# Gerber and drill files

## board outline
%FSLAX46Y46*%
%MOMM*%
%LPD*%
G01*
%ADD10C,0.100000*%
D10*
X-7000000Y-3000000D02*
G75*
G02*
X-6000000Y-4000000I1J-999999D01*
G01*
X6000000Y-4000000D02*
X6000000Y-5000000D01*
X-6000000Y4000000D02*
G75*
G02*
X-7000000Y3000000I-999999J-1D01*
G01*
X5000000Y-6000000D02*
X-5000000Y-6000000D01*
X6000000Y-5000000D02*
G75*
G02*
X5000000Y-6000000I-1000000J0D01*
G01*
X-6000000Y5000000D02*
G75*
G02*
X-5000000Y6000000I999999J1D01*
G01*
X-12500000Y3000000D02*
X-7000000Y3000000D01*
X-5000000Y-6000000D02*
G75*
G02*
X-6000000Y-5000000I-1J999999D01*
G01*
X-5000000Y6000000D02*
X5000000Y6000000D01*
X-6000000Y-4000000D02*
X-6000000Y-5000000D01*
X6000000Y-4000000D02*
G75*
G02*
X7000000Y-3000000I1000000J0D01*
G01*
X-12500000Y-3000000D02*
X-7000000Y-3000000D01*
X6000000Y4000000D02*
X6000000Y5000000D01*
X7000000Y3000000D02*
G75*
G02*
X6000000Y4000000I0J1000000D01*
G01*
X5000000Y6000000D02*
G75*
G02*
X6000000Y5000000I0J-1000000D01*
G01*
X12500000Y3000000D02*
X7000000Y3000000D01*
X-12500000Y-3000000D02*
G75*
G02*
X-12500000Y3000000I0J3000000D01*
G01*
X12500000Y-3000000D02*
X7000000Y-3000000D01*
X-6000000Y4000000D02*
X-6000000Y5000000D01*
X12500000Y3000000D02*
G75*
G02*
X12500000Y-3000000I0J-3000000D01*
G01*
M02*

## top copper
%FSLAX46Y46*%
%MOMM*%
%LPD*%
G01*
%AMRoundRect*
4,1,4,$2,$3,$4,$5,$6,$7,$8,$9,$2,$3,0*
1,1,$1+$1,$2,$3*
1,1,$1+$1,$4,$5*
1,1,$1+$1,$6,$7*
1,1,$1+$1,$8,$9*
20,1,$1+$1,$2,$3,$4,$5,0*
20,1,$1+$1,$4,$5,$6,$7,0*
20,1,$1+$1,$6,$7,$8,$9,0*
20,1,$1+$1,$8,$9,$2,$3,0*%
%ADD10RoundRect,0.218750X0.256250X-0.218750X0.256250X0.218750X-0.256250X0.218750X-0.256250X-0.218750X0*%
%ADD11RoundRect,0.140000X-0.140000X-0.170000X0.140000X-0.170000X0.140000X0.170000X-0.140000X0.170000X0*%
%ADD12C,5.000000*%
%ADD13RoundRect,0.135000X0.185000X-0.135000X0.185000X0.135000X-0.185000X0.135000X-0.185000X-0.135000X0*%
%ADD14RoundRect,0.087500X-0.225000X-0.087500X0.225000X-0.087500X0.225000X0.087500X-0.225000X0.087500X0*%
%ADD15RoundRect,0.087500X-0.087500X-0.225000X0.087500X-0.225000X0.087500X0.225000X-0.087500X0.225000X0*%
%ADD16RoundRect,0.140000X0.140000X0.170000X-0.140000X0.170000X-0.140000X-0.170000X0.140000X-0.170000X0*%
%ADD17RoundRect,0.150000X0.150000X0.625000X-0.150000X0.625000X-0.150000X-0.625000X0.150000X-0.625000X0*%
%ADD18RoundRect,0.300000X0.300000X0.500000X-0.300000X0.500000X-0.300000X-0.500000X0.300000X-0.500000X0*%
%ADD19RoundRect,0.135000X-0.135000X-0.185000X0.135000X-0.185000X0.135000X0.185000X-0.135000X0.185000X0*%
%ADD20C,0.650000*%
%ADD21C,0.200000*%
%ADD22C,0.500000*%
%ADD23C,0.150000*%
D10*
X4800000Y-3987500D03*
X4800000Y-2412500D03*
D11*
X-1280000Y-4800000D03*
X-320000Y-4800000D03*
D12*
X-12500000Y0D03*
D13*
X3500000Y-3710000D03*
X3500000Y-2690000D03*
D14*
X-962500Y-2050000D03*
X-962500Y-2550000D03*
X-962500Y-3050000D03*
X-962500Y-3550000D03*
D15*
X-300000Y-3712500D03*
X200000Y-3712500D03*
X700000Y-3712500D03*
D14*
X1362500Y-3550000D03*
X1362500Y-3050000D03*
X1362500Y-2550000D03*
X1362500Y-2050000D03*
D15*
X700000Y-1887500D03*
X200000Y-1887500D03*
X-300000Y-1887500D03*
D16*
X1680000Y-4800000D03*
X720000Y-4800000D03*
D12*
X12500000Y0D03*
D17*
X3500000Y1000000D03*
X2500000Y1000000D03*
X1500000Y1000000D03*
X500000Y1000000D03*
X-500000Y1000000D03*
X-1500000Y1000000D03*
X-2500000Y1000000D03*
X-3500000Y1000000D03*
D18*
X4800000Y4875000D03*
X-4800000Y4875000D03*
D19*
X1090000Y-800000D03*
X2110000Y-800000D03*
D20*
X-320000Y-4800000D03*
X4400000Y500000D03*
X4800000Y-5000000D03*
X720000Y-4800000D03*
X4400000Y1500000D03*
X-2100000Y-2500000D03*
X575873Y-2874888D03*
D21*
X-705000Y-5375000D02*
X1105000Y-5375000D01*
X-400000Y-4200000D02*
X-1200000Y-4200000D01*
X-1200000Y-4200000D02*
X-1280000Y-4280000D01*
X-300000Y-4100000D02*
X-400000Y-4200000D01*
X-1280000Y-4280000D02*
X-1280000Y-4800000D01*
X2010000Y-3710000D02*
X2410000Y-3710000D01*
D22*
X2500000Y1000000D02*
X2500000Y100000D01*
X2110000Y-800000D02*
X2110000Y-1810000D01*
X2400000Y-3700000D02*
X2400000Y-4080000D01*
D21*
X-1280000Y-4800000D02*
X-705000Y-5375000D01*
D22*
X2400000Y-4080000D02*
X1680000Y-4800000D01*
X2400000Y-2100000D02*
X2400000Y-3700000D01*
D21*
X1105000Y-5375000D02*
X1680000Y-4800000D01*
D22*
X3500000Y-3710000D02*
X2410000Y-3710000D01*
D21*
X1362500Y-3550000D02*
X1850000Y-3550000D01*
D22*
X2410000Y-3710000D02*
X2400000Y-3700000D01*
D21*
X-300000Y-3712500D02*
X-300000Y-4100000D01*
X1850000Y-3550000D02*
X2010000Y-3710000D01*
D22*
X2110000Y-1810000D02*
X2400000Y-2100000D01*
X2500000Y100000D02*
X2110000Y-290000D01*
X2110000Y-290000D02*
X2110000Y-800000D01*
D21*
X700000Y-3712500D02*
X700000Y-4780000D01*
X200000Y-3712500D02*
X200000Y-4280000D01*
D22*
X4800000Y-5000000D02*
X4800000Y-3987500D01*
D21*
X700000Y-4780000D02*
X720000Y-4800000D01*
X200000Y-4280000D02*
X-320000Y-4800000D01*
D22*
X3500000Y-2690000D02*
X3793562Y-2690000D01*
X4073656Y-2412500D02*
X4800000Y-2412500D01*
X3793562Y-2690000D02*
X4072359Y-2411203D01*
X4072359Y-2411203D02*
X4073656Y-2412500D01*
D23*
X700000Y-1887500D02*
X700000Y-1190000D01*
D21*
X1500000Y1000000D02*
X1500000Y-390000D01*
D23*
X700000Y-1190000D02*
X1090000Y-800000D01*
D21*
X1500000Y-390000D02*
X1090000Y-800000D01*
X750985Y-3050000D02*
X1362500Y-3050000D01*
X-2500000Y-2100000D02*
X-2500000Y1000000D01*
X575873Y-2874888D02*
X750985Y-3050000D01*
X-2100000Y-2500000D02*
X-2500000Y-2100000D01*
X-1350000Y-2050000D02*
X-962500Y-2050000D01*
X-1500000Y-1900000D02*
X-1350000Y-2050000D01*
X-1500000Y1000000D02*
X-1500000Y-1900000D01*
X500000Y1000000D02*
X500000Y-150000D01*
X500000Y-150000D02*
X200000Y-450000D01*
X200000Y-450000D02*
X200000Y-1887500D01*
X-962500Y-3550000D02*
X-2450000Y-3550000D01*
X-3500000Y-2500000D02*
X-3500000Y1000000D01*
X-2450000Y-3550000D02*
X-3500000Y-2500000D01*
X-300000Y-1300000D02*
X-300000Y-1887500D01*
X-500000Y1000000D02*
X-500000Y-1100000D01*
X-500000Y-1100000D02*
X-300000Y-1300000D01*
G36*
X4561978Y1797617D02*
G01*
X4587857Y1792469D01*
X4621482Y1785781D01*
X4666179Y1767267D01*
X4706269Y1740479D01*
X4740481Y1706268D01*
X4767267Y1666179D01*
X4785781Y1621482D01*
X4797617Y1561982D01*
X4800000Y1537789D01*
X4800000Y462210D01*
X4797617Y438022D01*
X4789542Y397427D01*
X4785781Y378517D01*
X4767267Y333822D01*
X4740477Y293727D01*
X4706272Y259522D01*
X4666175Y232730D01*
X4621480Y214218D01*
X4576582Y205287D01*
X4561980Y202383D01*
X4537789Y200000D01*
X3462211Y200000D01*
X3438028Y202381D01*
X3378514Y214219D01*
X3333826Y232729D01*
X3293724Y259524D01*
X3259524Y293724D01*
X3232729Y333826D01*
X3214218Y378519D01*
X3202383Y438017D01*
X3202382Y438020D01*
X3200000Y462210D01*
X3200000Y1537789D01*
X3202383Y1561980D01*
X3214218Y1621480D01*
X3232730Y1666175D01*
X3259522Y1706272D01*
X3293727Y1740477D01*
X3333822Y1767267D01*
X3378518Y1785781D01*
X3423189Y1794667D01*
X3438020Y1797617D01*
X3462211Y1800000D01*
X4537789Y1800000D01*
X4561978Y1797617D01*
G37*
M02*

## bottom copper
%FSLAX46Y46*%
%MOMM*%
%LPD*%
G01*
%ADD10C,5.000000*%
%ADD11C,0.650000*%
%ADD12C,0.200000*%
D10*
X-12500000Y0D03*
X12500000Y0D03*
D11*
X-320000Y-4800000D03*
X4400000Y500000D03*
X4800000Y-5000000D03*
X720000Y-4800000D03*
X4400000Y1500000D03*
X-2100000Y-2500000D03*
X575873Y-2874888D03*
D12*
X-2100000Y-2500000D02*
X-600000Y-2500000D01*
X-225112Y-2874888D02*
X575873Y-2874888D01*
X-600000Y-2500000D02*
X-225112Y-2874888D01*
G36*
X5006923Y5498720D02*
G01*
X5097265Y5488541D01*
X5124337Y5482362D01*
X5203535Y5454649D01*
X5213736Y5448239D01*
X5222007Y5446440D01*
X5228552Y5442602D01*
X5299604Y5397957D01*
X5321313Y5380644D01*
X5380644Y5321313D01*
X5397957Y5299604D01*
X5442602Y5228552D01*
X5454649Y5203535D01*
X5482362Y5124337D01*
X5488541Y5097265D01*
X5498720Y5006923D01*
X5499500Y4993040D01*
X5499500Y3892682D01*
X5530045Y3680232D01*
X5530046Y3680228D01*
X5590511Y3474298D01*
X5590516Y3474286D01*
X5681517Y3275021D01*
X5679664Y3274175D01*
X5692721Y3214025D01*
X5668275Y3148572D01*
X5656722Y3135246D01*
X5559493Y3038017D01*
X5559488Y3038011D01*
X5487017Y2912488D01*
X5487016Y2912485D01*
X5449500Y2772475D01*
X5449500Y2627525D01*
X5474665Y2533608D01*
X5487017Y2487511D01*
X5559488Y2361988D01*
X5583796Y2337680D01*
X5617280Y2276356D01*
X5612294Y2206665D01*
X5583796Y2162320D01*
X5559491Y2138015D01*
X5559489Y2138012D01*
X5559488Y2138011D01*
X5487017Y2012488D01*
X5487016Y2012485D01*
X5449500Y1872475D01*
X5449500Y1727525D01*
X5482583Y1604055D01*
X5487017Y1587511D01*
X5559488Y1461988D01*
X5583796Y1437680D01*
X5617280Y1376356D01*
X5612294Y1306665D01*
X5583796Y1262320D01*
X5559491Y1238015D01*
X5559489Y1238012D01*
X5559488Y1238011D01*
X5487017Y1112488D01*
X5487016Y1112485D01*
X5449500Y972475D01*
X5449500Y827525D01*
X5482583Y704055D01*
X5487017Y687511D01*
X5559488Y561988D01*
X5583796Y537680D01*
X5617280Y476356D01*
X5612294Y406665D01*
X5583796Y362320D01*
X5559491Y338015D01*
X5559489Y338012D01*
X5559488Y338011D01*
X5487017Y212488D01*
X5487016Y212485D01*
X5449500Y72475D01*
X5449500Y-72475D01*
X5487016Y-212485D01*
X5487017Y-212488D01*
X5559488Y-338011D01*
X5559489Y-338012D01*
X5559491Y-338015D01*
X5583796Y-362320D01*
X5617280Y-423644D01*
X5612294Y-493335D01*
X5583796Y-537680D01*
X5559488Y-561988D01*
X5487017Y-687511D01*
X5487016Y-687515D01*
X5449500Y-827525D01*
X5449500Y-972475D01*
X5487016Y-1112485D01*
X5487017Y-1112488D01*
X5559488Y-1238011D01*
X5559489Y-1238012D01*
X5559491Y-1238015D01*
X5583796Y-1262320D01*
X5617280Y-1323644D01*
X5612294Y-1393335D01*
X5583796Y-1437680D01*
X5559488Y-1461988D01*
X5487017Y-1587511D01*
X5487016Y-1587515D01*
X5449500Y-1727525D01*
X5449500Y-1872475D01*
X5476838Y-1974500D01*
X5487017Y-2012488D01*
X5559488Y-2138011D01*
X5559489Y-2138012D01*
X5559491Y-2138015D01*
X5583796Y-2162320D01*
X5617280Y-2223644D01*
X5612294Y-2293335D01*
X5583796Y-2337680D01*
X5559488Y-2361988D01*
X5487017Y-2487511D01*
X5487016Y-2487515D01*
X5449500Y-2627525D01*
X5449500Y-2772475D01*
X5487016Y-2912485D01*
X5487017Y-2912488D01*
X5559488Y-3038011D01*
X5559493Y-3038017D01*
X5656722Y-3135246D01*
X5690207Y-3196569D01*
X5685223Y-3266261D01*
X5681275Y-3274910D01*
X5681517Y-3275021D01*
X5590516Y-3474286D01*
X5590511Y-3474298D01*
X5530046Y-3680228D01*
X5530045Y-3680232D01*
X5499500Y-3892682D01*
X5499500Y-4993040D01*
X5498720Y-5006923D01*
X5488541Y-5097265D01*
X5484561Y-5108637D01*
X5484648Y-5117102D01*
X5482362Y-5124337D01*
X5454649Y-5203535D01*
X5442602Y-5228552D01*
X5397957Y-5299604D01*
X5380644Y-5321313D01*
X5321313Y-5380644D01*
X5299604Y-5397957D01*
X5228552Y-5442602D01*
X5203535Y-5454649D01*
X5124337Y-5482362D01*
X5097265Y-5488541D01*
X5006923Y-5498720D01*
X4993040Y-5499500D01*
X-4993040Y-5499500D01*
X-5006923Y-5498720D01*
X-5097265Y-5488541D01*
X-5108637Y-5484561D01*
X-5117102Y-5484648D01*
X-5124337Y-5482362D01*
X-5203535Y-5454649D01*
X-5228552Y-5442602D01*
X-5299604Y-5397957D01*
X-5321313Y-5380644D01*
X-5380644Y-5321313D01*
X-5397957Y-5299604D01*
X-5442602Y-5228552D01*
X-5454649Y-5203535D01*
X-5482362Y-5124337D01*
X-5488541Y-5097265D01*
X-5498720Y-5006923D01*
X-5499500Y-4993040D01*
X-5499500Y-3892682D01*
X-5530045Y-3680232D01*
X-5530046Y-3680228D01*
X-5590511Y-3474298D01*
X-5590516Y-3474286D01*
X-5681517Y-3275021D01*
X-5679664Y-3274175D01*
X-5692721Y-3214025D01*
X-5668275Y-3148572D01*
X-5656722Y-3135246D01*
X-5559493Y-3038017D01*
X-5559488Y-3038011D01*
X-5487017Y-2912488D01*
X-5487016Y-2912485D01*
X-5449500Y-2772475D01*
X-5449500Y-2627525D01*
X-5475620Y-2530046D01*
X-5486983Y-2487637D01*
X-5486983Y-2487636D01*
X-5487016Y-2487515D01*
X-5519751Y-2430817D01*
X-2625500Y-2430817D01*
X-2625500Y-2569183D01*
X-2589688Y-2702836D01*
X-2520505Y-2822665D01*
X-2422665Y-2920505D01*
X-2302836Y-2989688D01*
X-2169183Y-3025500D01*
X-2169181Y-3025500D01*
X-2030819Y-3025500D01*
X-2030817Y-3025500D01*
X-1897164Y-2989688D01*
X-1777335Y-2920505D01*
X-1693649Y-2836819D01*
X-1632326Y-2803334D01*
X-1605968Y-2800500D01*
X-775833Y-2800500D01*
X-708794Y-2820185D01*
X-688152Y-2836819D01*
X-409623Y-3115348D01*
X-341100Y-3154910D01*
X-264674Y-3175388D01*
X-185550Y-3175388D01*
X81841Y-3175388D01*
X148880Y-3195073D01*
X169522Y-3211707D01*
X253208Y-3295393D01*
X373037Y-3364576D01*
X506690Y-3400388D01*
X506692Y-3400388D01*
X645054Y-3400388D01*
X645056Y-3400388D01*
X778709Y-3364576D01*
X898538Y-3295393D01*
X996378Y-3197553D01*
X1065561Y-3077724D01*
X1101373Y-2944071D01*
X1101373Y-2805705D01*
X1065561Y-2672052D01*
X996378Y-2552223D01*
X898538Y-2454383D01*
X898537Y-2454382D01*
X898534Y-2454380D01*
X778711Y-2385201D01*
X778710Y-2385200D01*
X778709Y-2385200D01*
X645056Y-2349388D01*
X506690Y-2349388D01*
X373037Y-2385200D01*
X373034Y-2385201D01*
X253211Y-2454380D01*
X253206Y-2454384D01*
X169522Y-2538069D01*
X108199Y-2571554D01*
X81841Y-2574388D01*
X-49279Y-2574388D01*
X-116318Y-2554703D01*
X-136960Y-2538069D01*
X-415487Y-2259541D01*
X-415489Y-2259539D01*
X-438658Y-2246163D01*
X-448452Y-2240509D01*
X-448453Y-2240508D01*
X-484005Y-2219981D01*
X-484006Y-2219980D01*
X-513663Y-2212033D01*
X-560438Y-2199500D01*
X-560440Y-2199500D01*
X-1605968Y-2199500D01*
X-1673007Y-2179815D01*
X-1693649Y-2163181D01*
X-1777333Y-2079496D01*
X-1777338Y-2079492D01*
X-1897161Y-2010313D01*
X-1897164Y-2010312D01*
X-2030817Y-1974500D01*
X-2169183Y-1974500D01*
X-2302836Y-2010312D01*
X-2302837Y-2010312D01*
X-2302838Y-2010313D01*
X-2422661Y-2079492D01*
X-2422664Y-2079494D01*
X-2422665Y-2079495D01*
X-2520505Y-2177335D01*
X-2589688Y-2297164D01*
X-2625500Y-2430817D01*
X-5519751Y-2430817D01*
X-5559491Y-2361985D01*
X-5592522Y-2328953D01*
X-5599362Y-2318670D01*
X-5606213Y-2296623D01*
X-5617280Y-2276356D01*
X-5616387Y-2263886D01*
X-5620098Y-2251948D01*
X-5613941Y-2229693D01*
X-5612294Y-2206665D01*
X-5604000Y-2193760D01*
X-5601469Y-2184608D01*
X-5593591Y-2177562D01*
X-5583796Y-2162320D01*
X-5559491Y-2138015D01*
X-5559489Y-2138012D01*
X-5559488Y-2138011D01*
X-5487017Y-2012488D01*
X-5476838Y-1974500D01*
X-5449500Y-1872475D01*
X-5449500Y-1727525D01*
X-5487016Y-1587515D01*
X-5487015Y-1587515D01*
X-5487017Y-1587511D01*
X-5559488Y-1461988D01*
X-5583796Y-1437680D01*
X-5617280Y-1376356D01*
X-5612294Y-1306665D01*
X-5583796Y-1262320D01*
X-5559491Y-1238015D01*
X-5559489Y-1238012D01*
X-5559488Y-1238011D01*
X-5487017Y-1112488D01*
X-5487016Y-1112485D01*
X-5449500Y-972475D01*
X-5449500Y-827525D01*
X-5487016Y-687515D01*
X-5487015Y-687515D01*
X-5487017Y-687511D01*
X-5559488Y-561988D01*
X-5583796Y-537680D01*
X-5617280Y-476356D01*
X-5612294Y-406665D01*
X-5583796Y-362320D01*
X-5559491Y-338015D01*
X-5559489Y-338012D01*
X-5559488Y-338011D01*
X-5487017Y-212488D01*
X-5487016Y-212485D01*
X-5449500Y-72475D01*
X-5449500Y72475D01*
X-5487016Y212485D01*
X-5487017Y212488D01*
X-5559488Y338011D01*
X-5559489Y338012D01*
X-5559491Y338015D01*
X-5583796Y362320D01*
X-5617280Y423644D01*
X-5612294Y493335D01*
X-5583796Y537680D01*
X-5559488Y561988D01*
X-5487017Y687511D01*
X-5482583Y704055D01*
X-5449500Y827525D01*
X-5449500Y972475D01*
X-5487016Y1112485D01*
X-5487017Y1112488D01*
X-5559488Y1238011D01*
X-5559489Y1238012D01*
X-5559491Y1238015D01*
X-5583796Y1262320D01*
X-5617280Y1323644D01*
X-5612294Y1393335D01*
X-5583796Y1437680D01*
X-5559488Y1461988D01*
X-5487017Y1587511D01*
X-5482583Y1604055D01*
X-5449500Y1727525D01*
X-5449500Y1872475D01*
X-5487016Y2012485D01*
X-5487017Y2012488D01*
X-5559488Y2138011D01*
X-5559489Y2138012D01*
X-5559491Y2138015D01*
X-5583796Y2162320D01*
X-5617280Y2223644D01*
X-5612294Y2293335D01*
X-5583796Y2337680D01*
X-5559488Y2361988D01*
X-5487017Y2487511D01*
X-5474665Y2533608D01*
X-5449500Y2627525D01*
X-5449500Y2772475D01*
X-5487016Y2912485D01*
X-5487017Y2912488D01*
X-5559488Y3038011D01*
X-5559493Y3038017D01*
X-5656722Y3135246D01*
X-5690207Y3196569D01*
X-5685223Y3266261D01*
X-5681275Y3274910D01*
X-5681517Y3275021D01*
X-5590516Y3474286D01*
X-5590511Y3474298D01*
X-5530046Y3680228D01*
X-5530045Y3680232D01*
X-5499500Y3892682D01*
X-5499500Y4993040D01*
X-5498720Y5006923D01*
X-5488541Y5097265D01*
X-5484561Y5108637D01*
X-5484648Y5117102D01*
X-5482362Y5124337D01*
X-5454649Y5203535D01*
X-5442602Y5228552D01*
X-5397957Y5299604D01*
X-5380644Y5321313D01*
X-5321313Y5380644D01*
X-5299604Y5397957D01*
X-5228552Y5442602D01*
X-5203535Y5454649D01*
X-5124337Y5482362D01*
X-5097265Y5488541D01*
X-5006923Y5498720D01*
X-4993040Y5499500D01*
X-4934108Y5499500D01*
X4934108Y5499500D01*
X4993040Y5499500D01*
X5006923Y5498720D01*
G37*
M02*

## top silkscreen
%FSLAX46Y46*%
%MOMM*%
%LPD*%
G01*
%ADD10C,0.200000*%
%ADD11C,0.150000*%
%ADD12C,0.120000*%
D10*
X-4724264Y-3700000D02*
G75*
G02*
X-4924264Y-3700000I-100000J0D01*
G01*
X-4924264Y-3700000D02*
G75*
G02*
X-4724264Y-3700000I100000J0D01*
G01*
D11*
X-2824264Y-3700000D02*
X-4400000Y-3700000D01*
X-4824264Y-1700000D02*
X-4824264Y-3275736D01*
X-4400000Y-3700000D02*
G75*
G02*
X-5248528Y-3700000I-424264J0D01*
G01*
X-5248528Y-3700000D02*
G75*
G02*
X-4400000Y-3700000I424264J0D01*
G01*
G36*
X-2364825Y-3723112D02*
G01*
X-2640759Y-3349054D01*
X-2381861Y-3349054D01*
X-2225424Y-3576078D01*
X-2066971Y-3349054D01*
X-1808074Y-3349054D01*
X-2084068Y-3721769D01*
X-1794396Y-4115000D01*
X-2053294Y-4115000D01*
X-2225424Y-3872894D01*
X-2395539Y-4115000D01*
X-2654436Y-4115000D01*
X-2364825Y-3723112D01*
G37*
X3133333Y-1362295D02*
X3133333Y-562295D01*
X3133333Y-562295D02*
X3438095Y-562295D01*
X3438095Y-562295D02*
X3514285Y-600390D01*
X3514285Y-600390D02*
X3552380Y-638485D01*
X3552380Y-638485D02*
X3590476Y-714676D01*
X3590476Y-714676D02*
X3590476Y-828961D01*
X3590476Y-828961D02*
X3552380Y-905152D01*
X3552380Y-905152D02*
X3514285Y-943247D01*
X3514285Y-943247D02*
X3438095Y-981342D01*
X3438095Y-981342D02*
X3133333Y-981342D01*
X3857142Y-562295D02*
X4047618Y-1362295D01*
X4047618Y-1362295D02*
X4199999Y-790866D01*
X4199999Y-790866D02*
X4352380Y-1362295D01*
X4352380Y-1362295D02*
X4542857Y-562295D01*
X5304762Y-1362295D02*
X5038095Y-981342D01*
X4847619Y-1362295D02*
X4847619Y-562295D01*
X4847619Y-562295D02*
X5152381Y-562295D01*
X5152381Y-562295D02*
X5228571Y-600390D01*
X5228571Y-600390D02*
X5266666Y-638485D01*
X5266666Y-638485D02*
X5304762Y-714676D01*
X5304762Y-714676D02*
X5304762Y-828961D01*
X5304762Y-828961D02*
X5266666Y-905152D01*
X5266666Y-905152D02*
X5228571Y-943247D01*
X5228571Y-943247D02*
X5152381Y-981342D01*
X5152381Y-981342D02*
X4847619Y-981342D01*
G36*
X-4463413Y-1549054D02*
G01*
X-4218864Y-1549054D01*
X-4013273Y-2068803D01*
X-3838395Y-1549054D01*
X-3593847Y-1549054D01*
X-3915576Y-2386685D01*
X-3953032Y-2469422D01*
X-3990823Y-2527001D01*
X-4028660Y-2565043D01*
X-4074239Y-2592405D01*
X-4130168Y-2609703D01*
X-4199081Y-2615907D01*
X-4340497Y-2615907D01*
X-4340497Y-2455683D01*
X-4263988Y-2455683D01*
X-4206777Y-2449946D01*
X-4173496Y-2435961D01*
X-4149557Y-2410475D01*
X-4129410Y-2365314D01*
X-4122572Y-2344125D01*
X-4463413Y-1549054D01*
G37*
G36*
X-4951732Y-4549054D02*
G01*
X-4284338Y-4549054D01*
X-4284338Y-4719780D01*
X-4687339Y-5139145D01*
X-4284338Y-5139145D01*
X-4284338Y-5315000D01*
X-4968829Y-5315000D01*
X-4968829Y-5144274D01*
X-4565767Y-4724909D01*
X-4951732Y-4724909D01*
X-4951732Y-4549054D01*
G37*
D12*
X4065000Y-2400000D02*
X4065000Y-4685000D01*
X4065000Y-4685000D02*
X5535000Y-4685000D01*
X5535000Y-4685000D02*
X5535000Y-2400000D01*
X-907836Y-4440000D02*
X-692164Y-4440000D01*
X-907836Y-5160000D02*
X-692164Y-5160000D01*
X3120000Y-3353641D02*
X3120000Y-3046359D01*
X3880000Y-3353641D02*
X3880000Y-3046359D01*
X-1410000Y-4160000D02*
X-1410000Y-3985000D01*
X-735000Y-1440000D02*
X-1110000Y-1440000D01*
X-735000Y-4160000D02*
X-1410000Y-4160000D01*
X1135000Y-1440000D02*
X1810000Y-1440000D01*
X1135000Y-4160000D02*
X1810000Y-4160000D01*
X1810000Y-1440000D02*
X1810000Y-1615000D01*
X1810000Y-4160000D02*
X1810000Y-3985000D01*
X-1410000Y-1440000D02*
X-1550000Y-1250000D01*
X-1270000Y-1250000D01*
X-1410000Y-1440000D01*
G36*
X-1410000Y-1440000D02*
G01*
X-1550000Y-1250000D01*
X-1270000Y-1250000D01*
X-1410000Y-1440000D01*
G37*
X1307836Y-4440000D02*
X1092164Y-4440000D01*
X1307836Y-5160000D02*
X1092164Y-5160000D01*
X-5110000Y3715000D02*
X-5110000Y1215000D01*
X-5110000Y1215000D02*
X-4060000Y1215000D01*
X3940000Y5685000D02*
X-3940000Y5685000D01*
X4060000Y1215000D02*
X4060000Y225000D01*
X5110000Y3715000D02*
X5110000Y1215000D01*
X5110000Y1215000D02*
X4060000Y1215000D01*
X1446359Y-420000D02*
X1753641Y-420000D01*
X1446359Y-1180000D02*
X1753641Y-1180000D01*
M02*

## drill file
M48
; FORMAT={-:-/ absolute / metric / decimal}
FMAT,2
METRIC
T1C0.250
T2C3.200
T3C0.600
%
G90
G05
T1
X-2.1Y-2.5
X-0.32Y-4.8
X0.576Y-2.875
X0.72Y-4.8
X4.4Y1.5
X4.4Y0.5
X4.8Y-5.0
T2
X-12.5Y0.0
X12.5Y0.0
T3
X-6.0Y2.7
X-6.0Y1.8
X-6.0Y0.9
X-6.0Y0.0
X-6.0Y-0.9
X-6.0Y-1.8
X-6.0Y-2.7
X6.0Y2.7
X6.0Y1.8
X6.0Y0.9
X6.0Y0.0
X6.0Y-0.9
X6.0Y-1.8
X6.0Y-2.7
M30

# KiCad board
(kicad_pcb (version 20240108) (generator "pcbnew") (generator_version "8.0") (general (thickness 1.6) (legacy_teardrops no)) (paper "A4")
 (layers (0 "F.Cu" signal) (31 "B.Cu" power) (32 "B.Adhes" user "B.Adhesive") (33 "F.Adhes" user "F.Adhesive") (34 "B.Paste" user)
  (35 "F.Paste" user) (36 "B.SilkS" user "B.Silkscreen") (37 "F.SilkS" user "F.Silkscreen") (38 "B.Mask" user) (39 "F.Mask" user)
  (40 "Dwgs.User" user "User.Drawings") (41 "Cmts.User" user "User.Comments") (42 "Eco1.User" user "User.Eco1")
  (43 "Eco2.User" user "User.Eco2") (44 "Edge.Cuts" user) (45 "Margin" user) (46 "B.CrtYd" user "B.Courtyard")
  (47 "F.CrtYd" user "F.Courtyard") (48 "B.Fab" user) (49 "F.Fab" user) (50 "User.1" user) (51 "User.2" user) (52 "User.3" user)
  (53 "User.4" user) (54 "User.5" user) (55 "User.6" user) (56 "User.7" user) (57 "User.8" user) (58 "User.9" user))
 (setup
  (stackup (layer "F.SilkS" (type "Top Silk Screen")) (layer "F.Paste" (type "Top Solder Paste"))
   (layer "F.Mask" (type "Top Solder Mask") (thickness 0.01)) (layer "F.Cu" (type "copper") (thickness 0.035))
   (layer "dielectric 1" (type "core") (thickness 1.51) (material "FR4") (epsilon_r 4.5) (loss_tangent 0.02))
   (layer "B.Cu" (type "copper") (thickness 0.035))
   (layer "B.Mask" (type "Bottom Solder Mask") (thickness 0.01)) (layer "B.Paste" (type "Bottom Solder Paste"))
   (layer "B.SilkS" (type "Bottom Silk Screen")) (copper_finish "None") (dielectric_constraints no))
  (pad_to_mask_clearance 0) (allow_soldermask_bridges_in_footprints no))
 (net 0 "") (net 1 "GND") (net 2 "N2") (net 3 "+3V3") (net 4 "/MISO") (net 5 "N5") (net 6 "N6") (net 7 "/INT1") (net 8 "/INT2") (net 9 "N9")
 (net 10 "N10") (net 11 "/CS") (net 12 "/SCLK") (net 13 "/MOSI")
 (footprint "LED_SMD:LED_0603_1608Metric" (layer "F.Cu") (at 4.8 3.2 90)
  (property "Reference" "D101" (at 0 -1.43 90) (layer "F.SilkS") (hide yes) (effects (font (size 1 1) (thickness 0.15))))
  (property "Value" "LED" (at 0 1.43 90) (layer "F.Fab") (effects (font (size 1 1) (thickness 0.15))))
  (fp_line (start 0.8 -0.735) (end -1.485 -0.735) (stroke (width 0.12) (type solid)) (layer "F.SilkS"))
  (fp_line (start -1.485 -0.735) (end -1.485 0.735) (stroke (width 0.12) (type solid)) (layer "F.SilkS"))
  (fp_line (start -1.485 0.735) (end 0.8 0.735) (stroke (width 0.12) (type solid)) (layer "F.SilkS"))
  (pad "1" smd roundrect (at -0.7875 0 90) (size 0.875 0.95) (layers "F.Cu" "F.Paste" "F.Mask") (roundrect_rratio 0.25) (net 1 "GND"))
  (pad "2" smd roundrect (at 0.7875 0 90) (size 0.875 0.95) (layers "F.Cu" "F.Paste" "F.Mask") (roundrect_rratio 0.25) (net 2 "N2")))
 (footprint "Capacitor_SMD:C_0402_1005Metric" (layer "F.Cu") (at -0.8 4.8)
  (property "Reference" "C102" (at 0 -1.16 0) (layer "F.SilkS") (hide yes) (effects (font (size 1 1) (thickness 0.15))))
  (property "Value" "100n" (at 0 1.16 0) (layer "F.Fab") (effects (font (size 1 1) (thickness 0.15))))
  (fp_line (start -0.107836 -0.36) (end 0.107836 -0.36) (stroke (width 0.12) (type solid)) (layer "F.SilkS"))
  (fp_line (start -0.107836 0.36) (end 0.107836 0.36) (stroke (width 0.12) (type solid)) (layer "F.SilkS"))
  (pad "1" smd roundrect (at -0.48 0) (size 0.56 0.62) (layers "F.Cu" "F.Paste" "F.Mask") (roundrect_rratio 0.25) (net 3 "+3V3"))
  (pad "2" smd roundrect (at 0.48 0) (size 0.56 0.62) (layers "F.Cu" "F.Paste" "F.Mask") (roundrect_rratio 0.25) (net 1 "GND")))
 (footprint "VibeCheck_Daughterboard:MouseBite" (layer "F.Cu") (at -6 0 180)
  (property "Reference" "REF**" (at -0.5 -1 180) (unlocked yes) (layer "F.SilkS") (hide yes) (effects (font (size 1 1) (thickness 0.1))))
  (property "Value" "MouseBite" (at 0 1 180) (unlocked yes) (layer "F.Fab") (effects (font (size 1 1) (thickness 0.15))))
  (pad "" np_thru_hole circle (at 0 -2.7 180) (size 0.6 0.6) (drill 0.6) (layers "F&B.Cu"))
  (pad "" np_thru_hole circle (at 0 -1.8 180) (size 0.6 0.6) (drill 0.6) (layers "F&B.Cu"))
  (pad "" np_thru_hole circle (at 0 -0.9 180) (size 0.6 0.6) (drill 0.6) (layers "F&B.Cu"))
  (pad "" np_thru_hole circle (at 0 0 180) (size 0.6 0.6) (drill 0.6) (layers "F&B.Cu"))
  (pad "" np_thru_hole circle (at 0 0.9 180) (size 0.6 0.6) (drill 0.6) (layers "F&B.Cu"))
  (pad "" np_thru_hole circle (at 0 1.8 180) (size 0.6 0.6) (drill 0.6) (layers "F&B.Cu"))
  (pad "" np_thru_hole circle (at 0 2.7 180) (size 0.6 0.6) (drill 0.6) (layers "F&B.Cu")))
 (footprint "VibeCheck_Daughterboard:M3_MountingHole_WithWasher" (layer "F.Cu") (at -12.5 0)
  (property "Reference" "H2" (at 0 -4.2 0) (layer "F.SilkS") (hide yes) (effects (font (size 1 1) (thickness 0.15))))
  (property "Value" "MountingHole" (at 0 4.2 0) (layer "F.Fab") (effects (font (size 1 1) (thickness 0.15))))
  (pad "1" thru_hole circle (at 0 0) (size 5 5) (drill 3.2) (layers "*.Cu" "*.Mask") (remove_unused_layers no)))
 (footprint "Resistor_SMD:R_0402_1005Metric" (layer "F.Cu") (at 3.5 3.2 90)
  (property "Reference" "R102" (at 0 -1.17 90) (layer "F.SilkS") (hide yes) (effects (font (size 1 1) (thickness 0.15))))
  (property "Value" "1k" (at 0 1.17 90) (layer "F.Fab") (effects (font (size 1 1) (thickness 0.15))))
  (fp_line (start -0.153641 -0.38) (end 0.153641 -0.38) (stroke (width 0.12) (type solid)) (layer "F.SilkS"))
  (fp_line (start -0.153641 0.38) (end 0.153641 0.38) (stroke (width 0.12) (type solid)) (layer "F.SilkS"))
  (pad "1" smd roundrect (at -0.51 0 90) (size 0.54 0.64) (layers "F.Cu" "F.Paste" "F.Mask") (roundrect_rratio 0.25) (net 3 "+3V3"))
  (pad "2" smd roundrect (at 0.51 0 90) (size 0.54 0.64) (layers "F.Cu" "F.Paste" "F.Mask") (roundrect_rratio 0.25) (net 2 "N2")))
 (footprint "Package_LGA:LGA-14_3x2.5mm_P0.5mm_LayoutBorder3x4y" (layer "F.Cu") (at 0.2 2.8)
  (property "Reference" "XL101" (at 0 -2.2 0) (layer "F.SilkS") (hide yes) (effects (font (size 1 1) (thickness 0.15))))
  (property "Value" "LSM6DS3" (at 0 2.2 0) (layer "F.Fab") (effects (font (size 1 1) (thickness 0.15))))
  (fp_line (start -1.61 1.36) (end -1.61 1.185) (stroke (width 0.12) (type solid)) (layer "F.SilkS"))
  (fp_line (start -0.935 -1.36) (end -1.31 -1.36) (stroke (width 0.12) (type solid)) (layer "F.SilkS"))
  (fp_line (start -0.935 1.36) (end -1.61 1.36) (stroke (width 0.12) (type solid)) (layer "F.SilkS"))
  (fp_line (start 0.935 -1.36) (end 1.61 -1.36) (stroke (width 0.12) (type solid)) (layer "F.SilkS"))
  (fp_line (start 0.935 1.36) (end 1.61 1.36) (stroke (width 0.12) (type solid)) (layer "F.SilkS"))
  (fp_line (start 1.61 -1.36) (end 1.61 -1.185) (stroke (width 0.12) (type solid)) (layer "F.SilkS"))
  (fp_line (start 1.61 1.36) (end 1.61 1.185) (stroke (width 0.12) (type solid)) (layer "F.SilkS"))
  (fp_poly
   (pts (xy -1.61 -1.36) (xy -1.75 -1.55) (xy -1.47 -1.55) (xy -1.61 -1.36)) (stroke (width 0.12) (type solid)) (fill solid)
   (layer "F.SilkS"))
  (pad "1" smd roundrect (at -1.1625 -0.75) (size 0.625 0.35) (layers "F.Cu" "F.Paste" "F.Mask") (roundrect_rratio 0.25) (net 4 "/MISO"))
  (pad "2" smd roundrect (at -1.1625 -0.25) (size 0.625 0.35) (layers "F.Cu" "F.Paste" "F.Mask") (roundrect_rratio 0.25) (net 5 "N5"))
  (pad "3" smd roundrect (at -1.1625 0.25) (size 0.625 0.35) (layers "F.Cu" "F.Paste" "F.Mask") (roundrect_rratio 0.25) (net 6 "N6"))
  (pad "4" smd roundrect (at -1.1625 0.75) (size 0.625 0.35) (layers "F.Cu" "F.Paste" "F.Mask") (roundrect_rratio 0.25) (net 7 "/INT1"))
  (pad "5" smd roundrect (at -0.5 0.9125) (size 0.35 0.625) (layers "F.Cu" "F.Paste" "F.Mask") (roundrect_rratio 0.25) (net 3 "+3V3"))
  (pad "6" smd roundrect (at 0 0.9125) (size 0.35 0.625) (layers "F.Cu" "F.Paste" "F.Mask") (roundrect_rratio 0.25) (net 1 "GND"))
  (pad "7" smd roundrect (at 0.5 0.9125) (size 0.35 0.625) (layers "F.Cu" "F.Paste" "F.Mask") (roundrect_rratio 0.25) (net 1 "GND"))
  (pad "8" smd roundrect (at 1.1625 0.75) (size 0.625 0.35) (layers "F.Cu" "F.Paste" "F.Mask") (roundrect_rratio 0.25) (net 3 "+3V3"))
  (pad "9" smd roundrect (at 1.1625 0.25) (size 0.625 0.35) (layers "F.Cu" "F.Paste" "F.Mask") (roundrect_rratio 0.25) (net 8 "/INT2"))
  (pad "10" smd roundrect (at 1.1625 -0.25) (size 0.625 0.35) (layers "F.Cu" "F.Paste" "F.Mask") (roundrect_rratio 0.25) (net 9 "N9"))
  (pad "11" smd roundrect (at 1.1625 -0.75) (size 0.625 0.35) (layers "F.Cu" "F.Paste" "F.Mask") (roundrect_rratio 0.25) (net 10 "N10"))
  (pad "12" smd roundrect (at 0.5 -0.9125) (size 0.35 0.625) (layers "F.Cu" "F.Paste" "F.Mask") (roundrect_rratio 0.25) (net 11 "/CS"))
  (pad "13" smd roundrect (at 0 -0.9125) (size 0.35 0.625) (layers "F.Cu" "F.Paste" "F.Mask") (roundrect_rratio 0.25) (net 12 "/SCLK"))
  (pad "14" smd roundrect (at -0.5 -0.9125) (size 0.35 0.625) (layers "F.Cu" "F.Paste" "F.Mask") (roundrect_rratio 0.25) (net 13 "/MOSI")))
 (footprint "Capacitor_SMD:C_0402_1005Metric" (layer "F.Cu") (at 1.2 4.8 180)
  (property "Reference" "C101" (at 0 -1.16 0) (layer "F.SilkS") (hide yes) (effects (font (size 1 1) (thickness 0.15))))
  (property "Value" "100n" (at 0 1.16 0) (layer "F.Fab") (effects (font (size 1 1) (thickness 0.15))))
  (fp_line (start -0.107836 0.36) (end 0.107836 0.36) (stroke (width 0.12) (type solid)) (layer "F.SilkS"))
  (fp_line (start -0.107836 -0.36) (end 0.107836 -0.36) (stroke (width 0.12) (type solid)) (layer "F.SilkS"))
  (pad "1" smd roundrect (at -0.48 0 180) (size 0.56 0.62) (layers "F.Cu" "F.Paste" "F.Mask") (roundrect_rratio 0.25) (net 3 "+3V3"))
  (pad "2" smd roundrect (at 0.48 0 180) (size 0.56 0.62) (layers "F.Cu" "F.Paste" "F.Mask") (roundrect_rratio 0.25) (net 1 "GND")))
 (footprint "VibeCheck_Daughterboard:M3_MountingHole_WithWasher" (layer "F.Cu") (at 12.5 0)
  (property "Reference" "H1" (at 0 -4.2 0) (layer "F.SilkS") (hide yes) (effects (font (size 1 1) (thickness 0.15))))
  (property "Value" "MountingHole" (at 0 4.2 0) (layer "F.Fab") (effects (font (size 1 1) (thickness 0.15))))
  (pad "1" thru_hole circle (at 0 0) (size 5 5) (drill 3.2) (layers "*.Cu" "*.Mask") (remove_unused_layers no)))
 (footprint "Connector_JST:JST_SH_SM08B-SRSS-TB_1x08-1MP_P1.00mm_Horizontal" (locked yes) (layer "F.Cu") (at 0 -3 180)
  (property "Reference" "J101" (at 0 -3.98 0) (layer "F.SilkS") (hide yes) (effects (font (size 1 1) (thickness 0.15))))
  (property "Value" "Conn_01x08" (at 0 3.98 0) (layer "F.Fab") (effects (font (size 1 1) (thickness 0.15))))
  (fp_line (start 5.11 0.715) (end 5.11 -1.785) (stroke (width 0.12) (type solid)) (layer "F.SilkS"))
  (fp_line (start 5.11 -1.785) (end 4.06 -1.785) (stroke (width 0.12) (type solid)) (layer "F.SilkS"))
  (fp_line (start -3.94 2.685) (end 3.94 2.685) (stroke (width 0.12) (type solid)) (layer "F.SilkS"))
  (fp_line (start -4.06 -1.785) (end -4.06 -2.775) (stroke (width 0.12) (type solid)) (layer "F.SilkS"))
  (fp_line (start -5.11 0.715) (end -5.11 -1.785) (stroke (width 0.12) (type solid)) (layer "F.SilkS"))
  (fp_line (start -5.11 -1.785) (end -4.06 -1.785) (stroke (width 0.12) (type solid)) (layer "F.SilkS"))
  (pad "1" smd roundrect (at -3.5 -2 180) (size 0.6 1.55) (layers "F.Cu" "F.Paste" "F.Mask") (roundrect_rratio 0.25) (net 1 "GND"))
  (pad "2" smd roundrect (at -2.5 -2 180) (size 0.6 1.55) (layers "F.Cu" "F.Paste" "F.Mask") (roundrect_rratio 0.25) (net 3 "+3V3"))
  (pad "3" smd roundrect (at -1.5 -2 180) (size 0.6 1.55) (layers "F.Cu" "F.Paste" "F.Mask") (roundrect_rratio 0.25) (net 11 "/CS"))
  (pad "4" smd roundrect (at -0.5 -2 180) (size 0.6 1.55) (layers "F.Cu" "F.Paste" "F.Mask") (roundrect_rratio 0.25) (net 12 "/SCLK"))
  (pad "5" smd roundrect (at 0.5 -2 180) (size 0.6 1.55) (layers "F.Cu" "F.Paste" "F.Mask") (roundrect_rratio 0.25) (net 13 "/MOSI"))
  (pad "6" smd roundrect (at 1.5 -2 180) (size 0.6 1.55) (layers "F.Cu" "F.Paste" "F.Mask") (roundrect_rratio 0.25) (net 4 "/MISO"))
  (pad "7" smd roundrect (at 2.5 -2 180) (size 0.6 1.55) (layers "F.Cu" "F.Paste" "F.Mask") (roundrect_rratio 0.25) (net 8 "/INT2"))
  (pad "8" smd roundrect (at 3.5 -2 180) (size 0.6 1.55) (layers "F.Cu" "F.Paste" "F.Mask") (roundrect_rratio 0.25) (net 7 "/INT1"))
  (pad "MP" smd roundrect (at -4.8 1.875 180) (size 1.2 1.6) (layers "F.Cu" "F.Paste" "F.Mask") (roundrect_rratio 0.25))
  (pad "MP" smd roundrect (at 4.8 1.875 180) (size 1.2 1.6) (layers "F.Cu" "F.Paste" "F.Mask") (roundrect_rratio 0.25)))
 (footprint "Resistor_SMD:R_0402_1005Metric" (layer "F.Cu") (at 1.6 0.8)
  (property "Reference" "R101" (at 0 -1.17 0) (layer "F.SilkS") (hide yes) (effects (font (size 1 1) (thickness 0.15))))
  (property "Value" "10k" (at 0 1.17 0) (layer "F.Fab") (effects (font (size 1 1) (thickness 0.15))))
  (fp_line (start -0.153641 -0.38) (end 0.153641 -0.38) (stroke (width 0.12) (type solid)) (layer "F.SilkS"))
  (fp_line (start -0.153641 0.38) (end 0.153641 0.38) (stroke (width 0.12) (type solid)) (layer "F.SilkS"))
  (pad "1" smd roundrect (at -0.51 0) (size 0.54 0.64) (layers "F.Cu" "F.Paste" "F.Mask") (roundrect_rratio 0.25) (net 11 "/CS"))
  (pad "2" smd roundrect (at 0.51 0) (size 0.54 0.64) (layers "F.Cu" "F.Paste" "F.Mask") (roundrect_rratio 0.25) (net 3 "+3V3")))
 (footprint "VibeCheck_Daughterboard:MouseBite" (layer "F.Cu") (at 6 0)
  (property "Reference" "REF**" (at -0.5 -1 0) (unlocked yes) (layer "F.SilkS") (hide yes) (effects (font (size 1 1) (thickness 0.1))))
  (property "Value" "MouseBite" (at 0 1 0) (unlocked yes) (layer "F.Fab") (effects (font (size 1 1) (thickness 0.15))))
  (pad "" np_thru_hole circle (at 0 -2.7) (size 0.6 0.6) (drill 0.6) (layers "F&B.Cu"))
  (pad "" np_thru_hole circle (at 0 -1.8) (size 0.6 0.6) (drill 0.6) (layers "F&B.Cu"))
  (pad "" np_thru_hole circle (at 0 -0.9) (size 0.6 0.6) (drill 0.6) (layers "F&B.Cu"))
  (pad "" np_thru_hole circle (at 0 0) (size 0.6 0.6) (drill 0.6) (layers "F&B.Cu"))
  (pad "" np_thru_hole circle (at 0 0.9) (size 0.6 0.6) (drill 0.6) (layers "F&B.Cu"))
  (pad "" np_thru_hole circle (at 0 1.8) (size 0.6 0.6) (drill 0.6) (layers "F&B.Cu"))
  (pad "" np_thru_hole circle (at 0 2.7) (size 0.6 0.6) (drill 0.6) (layers "F&B.Cu")))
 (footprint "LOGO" (layer "B.Cu") (at 0 -2 180)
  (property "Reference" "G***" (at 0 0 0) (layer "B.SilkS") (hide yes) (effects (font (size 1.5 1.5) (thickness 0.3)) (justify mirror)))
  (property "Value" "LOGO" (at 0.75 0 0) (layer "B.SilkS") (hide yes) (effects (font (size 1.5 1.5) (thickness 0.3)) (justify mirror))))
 (gr_circle (center -4.824264 3.7) (end -4.824264 3.8) (stroke (width 0.2) (type default)) (fill none) (layer "F.SilkS"))
 (gr_line (start -2.824264 3.7) (end -4.4 3.7) (stroke (width 0.15) (type default)) (layer "F.SilkS"))
 (gr_line (start -4.824264 1.7) (end -4.824264 3.275736) (stroke (width 0.15) (type default)) (layer "F.SilkS"))
 (gr_circle (center -4.824264 3.7) (end -4.524264 3.4) (stroke (width 0.15) (type default)) (fill none) (layer "F.SilkS"))
 (gr_arc (start -7 3) (mid -6.292893 3.292893) (end -6 4) (stroke (width 0.1) (type default)) (layer "Edge.Cuts"))
 (gr_line (start 6 4) (end 6 5) (stroke (width 0.1) (type default)) (layer "Edge.Cuts"))
 (gr_arc (start -6 -4) (mid -6.292893 -3.292893) (end -7 -3) (stroke (width 0.1) (type default)) (layer "Edge.Cuts"))
 (gr_line (start 5 6) (end -5 6) (stroke (width 0.1) (type default)) (layer "Edge.Cuts"))
 (gr_arc (start 6 5) (mid 5.707107 5.707107) (end 5 6) (stroke (width 0.1) (type default)) (layer "Edge.Cuts"))
 (gr_arc (start -6 -5) (mid -5.707107 -5.707107) (end -5 -6) (stroke (width 0.1) (type default)) (layer "Edge.Cuts"))
 (gr_line (start -12.5 -3) (end -7 -3) (stroke (width 0.1) (type default)) (layer "Edge.Cuts"))
 (gr_arc (start -5 6) (mid -5.707107 5.707107) (end -6 5) (stroke (width 0.1) (type default)) (layer "Edge.Cuts"))
 (gr_line (start -5 -6) (end 5 -6) (stroke (width 0.1) (type default)) (layer "Edge.Cuts"))
 (gr_line (start -6 4) (end -6 5) (stroke (width 0.1) (type default)) (layer "Edge.Cuts"))
 (gr_arc (start 6 4) (mid 6.292893 3.292893) (end 7 3) (stroke (width 0.1) (type default)) (layer "Edge.Cuts"))
 (gr_line (start -12.5 3) (end -7 3) (stroke (width 0.1) (type default)) (layer "Edge.Cuts"))
 (gr_line (start 6 -4) (end 6 -5) (stroke (width 0.1) (type default)) (layer "Edge.Cuts"))
 (gr_arc (start 7 -3) (mid 6.292893 -3.292893) (end 6 -4) (stroke (width 0.1) (type default)) (layer "Edge.Cuts"))
 (gr_arc (start 5 -6) (mid 5.707107 -5.707107) (end 6 -5) (stroke (width 0.1) (type default)) (layer "Edge.Cuts"))
 (gr_line (start 12.5 -3) (end 7 -3) (stroke (width 0.1) (type default)) (layer "Edge.Cuts"))
 (gr_arc (start -12.5 3) (mid -15.5 0) (end -12.5 -3) (stroke (width 0.1) (type default)) (layer "Edge.Cuts"))
 (gr_line (start 12.5 3) (end 7 3) (stroke (width 0.1) (type default)) (layer "Edge.Cuts"))
 (gr_line (start -6 -4) (end -6 -5) (stroke (width 0.1) (type default)) (layer "Edge.Cuts"))
 (gr_arc (start 12.5 -3) (mid 15.5 0) (end 12.5 3) (stroke (width 0.1) (type default)) (layer "Edge.Cuts"))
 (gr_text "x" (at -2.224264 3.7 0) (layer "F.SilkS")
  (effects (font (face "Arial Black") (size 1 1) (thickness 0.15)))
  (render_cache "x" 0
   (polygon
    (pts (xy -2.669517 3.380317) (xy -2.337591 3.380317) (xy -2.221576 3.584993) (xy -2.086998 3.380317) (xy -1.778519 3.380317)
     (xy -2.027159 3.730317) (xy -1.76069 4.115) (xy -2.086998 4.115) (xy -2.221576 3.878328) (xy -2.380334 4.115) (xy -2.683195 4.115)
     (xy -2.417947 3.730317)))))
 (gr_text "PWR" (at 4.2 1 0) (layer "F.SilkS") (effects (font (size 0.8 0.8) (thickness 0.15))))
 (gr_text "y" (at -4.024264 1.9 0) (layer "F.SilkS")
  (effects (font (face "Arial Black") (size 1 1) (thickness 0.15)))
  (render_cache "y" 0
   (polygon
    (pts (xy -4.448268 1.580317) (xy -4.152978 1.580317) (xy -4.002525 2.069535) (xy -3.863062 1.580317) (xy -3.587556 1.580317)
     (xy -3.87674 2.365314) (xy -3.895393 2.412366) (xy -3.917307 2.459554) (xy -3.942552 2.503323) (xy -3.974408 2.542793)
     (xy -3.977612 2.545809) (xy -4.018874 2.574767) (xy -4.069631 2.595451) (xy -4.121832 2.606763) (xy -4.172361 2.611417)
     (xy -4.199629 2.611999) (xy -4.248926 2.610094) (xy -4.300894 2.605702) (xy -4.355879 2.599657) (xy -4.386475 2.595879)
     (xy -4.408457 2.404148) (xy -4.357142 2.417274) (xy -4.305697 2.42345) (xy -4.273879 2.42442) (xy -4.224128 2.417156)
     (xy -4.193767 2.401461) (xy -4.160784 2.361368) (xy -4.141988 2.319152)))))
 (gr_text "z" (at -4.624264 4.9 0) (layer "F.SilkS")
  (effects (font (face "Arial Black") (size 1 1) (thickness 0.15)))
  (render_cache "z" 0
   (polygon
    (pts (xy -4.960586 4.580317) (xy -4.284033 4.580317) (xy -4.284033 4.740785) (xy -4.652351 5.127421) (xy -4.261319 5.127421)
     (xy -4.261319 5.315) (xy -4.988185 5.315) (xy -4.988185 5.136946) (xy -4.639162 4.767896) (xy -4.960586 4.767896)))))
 (segment (start -0.705 5.375) (end 1.105 5.375) (width 0.2) (layer "F.Cu") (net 3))
 (segment (start -0.4 4.2) (end -1.2 4.2) (width 0.2) (layer "F.Cu") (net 3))
 (segment (start -1.2 4.2) (end -1.28 4.28) (width 0.2) (layer "F.Cu") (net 3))
 (segment (start -0.3 4.1) (end -0.4 4.2) (width 0.2) (layer "F.Cu") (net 3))
 (segment (start -1.28 4.28) (end -1.28 4.8) (width 0.2) (layer "F.Cu") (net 3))
 (segment (start 2.01 3.71) (end 2.41 3.71) (width 0.2) (layer "F.Cu") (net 3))
 (segment (start 2.5 -1) (end 2.5 -0.1) (width 0.5) (layer "F.Cu") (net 3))
 (segment (start 2.11 0.8) (end 2.11 1.81) (width 0.5) (layer "F.Cu") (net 3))
 (segment (start 2.4 3.7) (end 2.4 4.08) (width 0.5) (layer "F.Cu") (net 3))
 (segment (start -1.28 4.8) (end -0.705 5.375) (width 0.2) (layer "F.Cu") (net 3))
 (segment (start 2.4 4.08) (end 1.68 4.8) (width 0.5) (layer "F.Cu") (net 3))
 (segment (start 2.4 2.1) (end 2.4 3.7) (width 0.5) (layer "F.Cu") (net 3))
 (segment (start 1.105 5.375) (end 1.68 4.8) (width 0.2) (layer "F.Cu") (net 3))
 (segment (start 3.5 3.71) (end 2.41 3.71) (width 0.5) (layer "F.Cu") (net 3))
 (segment (start 1.3625 3.55) (end 1.85 3.55) (width 0.2) (layer "F.Cu") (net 3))
 (segment (start 2.41 3.71) (end 2.4 3.7) (width 0.5) (layer "F.Cu") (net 3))
 (segment (start -0.3 3.7125) (end -0.3 4.1) (width 0.2) (layer "F.Cu") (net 3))
 (segment (start 1.85 3.55) (end 2.01 3.71) (width 0.2) (layer "F.Cu") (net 3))
 (segment (start 2.11 1.81) (end 2.4 2.1) (width 0.5) (layer "F.Cu") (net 3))
 (segment (start 2.5 -0.1) (end 2.11 0.29) (width 0.5) (layer "F.Cu") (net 3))
 (segment (start 2.11 0.29) (end 2.11 0.8) (width 0.5) (layer "F.Cu") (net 3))
 (segment (start 0.7 3.7125) (end 0.7 4.78) (width 0.2) (layer "F.Cu") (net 1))
 (segment (start 0.2 3.7125) (end 0.2 4.28) (width 0.2) (layer "F.Cu") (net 1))
 (segment (start 4.8 5) (end 4.8 3.9875) (width 0.5) (layer "F.Cu") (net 1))
 (segment (start 0.7 4.78) (end 0.72 4.8) (width 0.2) (layer "F.Cu") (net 1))
 (segment (start 0.2 4.28) (end -0.32 4.8) (width 0.2) (layer "F.Cu") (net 1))
 (via (at -0.32 4.8) (size 0.65) (drill 0.25) (layers "F.Cu" "B.Cu") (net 1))
 (via (at 4.4 -0.5) (size 0.65) (drill 0.25) (layers "F.Cu" "B.Cu") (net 1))
 (via (at 4.8 5) (size 0.65) (drill 0.25) (layers "F.Cu" "B.Cu") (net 1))
 (via (at 0.72 4.8) (size 0.65) (drill 0.25) (layers "F.Cu" "B.Cu") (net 1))
 (via (at 4.4 -1.5) (size 0.65) (drill 0.25) (layers "F.Cu" "B.Cu") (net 1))
 (segment (start 3.5 2.69) (end 3.793562 2.69) (width 0.5) (layer "F.Cu") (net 2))
 (segment (start 4.073656 2.4125) (end 4.8 2.4125) (width 0.5) (layer "F.Cu") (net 2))
 (segment (start 3.793562 2.69) (end 4.072359 2.411203) (width 0.5) (layer "F.Cu") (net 2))
 (segment (start 4.072359 2.411203) (end 4.073656 2.4125) (width 0.5) (layer "F.Cu") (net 2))
 (segment (start 0.7 1.8875) (end 0.7 1.19) (width 0.15) (layer "F.Cu") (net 11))
 (segment (start 1.5 -1) (end 1.5 0.39) (width 0.2) (layer "F.Cu") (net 11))
 (segment (start 0.7 1.19) (end 1.09 0.8) (width 0.15) (layer "F.Cu") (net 11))
 (segment (start 1.5 0.39) (end 1.09 0.8) (width 0.2) (layer "F.Cu") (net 11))
 (segment (start 0.750985 3.05) (end 1.3625 3.05) (width 0.2) (layer "F.Cu") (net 8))
 (segment (start -2.5 2.1) (end -2.5 -1) (width 0.2) (layer "F.Cu") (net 8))
 (segment (start 0.575873 2.874888) (end 0.750985 3.05) (width 0.2) (layer "F.Cu") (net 8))
 (segment (start -2.1 2.5) (end -2.5 2.1) (width 0.2) (layer "F.Cu") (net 8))
 (via (at -2.1 2.5) (size 0.65) (drill 0.25) (layers "F.Cu" "B.Cu") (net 8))
 (via (at 0.575873 2.874888) (size 0.65) (drill 0.25) (layers "F.Cu" "B.Cu") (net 8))
 (segment (start -2.1 2.5) (end -0.6 2.5) (width 0.2) (layer "B.Cu") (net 8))
 (segment (start -0.225112 2.874888) (end 0.575873 2.874888) (width 0.2) (layer "B.Cu") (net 8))
 (segment (start -0.6 2.5) (end -0.225112 2.874888) (width 0.2) (layer "B.Cu") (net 8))
 (segment (start -1.35 2.05) (end -0.9625 2.05) (width 0.2) (layer "F.Cu") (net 4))
 (segment (start -1.5 1.9) (end -1.35 2.05) (width 0.2) (layer "F.Cu") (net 4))
 (segment (start -1.5 -1) (end -1.5 1.9) (width 0.2) (layer "F.Cu") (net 4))
 (segment (start 0.5 -1) (end 0.5 0.15) (width 0.2) (layer "F.Cu") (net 12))
 (segment (start 0.5 0.15) (end 0.2 0.45) (width 0.2) (layer "F.Cu") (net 12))
 (segment (start 0.2 0.45) (end 0.2 1.8875) (width 0.2) (layer "F.Cu") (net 12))
 (segment (start -0.9625 3.55) (end -2.45 3.55) (width 0.2) (layer "F.Cu") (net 7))
 (segment (start -3.5 2.5) (end -3.5 -1) (width 0.2) (layer "F.Cu") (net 7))
 (segment (start -2.45 3.55) (end -3.5 2.5) (width 0.2) (layer "F.Cu") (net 7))
 (segment (start -0.3 1.3) (end -0.3 1.8875) (width 0.2) (layer "F.Cu") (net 13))
 (segment (start -0.5 -1) (end -0.5 1.1) (width 0.2) (layer "F.Cu") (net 13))
 (segment (start -0.5 1.1) (end -0.3 1.3) (width 0.2) (layer "F.Cu") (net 13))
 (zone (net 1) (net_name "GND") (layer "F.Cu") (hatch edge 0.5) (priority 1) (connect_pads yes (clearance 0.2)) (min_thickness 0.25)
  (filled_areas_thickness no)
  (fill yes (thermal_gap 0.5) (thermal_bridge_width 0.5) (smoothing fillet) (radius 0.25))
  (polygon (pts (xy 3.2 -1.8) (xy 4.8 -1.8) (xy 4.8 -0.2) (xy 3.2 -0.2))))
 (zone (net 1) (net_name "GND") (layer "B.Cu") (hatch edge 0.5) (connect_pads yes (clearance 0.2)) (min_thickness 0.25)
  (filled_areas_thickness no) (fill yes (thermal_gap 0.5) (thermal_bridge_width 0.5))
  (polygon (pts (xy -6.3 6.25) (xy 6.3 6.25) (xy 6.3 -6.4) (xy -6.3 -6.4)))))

